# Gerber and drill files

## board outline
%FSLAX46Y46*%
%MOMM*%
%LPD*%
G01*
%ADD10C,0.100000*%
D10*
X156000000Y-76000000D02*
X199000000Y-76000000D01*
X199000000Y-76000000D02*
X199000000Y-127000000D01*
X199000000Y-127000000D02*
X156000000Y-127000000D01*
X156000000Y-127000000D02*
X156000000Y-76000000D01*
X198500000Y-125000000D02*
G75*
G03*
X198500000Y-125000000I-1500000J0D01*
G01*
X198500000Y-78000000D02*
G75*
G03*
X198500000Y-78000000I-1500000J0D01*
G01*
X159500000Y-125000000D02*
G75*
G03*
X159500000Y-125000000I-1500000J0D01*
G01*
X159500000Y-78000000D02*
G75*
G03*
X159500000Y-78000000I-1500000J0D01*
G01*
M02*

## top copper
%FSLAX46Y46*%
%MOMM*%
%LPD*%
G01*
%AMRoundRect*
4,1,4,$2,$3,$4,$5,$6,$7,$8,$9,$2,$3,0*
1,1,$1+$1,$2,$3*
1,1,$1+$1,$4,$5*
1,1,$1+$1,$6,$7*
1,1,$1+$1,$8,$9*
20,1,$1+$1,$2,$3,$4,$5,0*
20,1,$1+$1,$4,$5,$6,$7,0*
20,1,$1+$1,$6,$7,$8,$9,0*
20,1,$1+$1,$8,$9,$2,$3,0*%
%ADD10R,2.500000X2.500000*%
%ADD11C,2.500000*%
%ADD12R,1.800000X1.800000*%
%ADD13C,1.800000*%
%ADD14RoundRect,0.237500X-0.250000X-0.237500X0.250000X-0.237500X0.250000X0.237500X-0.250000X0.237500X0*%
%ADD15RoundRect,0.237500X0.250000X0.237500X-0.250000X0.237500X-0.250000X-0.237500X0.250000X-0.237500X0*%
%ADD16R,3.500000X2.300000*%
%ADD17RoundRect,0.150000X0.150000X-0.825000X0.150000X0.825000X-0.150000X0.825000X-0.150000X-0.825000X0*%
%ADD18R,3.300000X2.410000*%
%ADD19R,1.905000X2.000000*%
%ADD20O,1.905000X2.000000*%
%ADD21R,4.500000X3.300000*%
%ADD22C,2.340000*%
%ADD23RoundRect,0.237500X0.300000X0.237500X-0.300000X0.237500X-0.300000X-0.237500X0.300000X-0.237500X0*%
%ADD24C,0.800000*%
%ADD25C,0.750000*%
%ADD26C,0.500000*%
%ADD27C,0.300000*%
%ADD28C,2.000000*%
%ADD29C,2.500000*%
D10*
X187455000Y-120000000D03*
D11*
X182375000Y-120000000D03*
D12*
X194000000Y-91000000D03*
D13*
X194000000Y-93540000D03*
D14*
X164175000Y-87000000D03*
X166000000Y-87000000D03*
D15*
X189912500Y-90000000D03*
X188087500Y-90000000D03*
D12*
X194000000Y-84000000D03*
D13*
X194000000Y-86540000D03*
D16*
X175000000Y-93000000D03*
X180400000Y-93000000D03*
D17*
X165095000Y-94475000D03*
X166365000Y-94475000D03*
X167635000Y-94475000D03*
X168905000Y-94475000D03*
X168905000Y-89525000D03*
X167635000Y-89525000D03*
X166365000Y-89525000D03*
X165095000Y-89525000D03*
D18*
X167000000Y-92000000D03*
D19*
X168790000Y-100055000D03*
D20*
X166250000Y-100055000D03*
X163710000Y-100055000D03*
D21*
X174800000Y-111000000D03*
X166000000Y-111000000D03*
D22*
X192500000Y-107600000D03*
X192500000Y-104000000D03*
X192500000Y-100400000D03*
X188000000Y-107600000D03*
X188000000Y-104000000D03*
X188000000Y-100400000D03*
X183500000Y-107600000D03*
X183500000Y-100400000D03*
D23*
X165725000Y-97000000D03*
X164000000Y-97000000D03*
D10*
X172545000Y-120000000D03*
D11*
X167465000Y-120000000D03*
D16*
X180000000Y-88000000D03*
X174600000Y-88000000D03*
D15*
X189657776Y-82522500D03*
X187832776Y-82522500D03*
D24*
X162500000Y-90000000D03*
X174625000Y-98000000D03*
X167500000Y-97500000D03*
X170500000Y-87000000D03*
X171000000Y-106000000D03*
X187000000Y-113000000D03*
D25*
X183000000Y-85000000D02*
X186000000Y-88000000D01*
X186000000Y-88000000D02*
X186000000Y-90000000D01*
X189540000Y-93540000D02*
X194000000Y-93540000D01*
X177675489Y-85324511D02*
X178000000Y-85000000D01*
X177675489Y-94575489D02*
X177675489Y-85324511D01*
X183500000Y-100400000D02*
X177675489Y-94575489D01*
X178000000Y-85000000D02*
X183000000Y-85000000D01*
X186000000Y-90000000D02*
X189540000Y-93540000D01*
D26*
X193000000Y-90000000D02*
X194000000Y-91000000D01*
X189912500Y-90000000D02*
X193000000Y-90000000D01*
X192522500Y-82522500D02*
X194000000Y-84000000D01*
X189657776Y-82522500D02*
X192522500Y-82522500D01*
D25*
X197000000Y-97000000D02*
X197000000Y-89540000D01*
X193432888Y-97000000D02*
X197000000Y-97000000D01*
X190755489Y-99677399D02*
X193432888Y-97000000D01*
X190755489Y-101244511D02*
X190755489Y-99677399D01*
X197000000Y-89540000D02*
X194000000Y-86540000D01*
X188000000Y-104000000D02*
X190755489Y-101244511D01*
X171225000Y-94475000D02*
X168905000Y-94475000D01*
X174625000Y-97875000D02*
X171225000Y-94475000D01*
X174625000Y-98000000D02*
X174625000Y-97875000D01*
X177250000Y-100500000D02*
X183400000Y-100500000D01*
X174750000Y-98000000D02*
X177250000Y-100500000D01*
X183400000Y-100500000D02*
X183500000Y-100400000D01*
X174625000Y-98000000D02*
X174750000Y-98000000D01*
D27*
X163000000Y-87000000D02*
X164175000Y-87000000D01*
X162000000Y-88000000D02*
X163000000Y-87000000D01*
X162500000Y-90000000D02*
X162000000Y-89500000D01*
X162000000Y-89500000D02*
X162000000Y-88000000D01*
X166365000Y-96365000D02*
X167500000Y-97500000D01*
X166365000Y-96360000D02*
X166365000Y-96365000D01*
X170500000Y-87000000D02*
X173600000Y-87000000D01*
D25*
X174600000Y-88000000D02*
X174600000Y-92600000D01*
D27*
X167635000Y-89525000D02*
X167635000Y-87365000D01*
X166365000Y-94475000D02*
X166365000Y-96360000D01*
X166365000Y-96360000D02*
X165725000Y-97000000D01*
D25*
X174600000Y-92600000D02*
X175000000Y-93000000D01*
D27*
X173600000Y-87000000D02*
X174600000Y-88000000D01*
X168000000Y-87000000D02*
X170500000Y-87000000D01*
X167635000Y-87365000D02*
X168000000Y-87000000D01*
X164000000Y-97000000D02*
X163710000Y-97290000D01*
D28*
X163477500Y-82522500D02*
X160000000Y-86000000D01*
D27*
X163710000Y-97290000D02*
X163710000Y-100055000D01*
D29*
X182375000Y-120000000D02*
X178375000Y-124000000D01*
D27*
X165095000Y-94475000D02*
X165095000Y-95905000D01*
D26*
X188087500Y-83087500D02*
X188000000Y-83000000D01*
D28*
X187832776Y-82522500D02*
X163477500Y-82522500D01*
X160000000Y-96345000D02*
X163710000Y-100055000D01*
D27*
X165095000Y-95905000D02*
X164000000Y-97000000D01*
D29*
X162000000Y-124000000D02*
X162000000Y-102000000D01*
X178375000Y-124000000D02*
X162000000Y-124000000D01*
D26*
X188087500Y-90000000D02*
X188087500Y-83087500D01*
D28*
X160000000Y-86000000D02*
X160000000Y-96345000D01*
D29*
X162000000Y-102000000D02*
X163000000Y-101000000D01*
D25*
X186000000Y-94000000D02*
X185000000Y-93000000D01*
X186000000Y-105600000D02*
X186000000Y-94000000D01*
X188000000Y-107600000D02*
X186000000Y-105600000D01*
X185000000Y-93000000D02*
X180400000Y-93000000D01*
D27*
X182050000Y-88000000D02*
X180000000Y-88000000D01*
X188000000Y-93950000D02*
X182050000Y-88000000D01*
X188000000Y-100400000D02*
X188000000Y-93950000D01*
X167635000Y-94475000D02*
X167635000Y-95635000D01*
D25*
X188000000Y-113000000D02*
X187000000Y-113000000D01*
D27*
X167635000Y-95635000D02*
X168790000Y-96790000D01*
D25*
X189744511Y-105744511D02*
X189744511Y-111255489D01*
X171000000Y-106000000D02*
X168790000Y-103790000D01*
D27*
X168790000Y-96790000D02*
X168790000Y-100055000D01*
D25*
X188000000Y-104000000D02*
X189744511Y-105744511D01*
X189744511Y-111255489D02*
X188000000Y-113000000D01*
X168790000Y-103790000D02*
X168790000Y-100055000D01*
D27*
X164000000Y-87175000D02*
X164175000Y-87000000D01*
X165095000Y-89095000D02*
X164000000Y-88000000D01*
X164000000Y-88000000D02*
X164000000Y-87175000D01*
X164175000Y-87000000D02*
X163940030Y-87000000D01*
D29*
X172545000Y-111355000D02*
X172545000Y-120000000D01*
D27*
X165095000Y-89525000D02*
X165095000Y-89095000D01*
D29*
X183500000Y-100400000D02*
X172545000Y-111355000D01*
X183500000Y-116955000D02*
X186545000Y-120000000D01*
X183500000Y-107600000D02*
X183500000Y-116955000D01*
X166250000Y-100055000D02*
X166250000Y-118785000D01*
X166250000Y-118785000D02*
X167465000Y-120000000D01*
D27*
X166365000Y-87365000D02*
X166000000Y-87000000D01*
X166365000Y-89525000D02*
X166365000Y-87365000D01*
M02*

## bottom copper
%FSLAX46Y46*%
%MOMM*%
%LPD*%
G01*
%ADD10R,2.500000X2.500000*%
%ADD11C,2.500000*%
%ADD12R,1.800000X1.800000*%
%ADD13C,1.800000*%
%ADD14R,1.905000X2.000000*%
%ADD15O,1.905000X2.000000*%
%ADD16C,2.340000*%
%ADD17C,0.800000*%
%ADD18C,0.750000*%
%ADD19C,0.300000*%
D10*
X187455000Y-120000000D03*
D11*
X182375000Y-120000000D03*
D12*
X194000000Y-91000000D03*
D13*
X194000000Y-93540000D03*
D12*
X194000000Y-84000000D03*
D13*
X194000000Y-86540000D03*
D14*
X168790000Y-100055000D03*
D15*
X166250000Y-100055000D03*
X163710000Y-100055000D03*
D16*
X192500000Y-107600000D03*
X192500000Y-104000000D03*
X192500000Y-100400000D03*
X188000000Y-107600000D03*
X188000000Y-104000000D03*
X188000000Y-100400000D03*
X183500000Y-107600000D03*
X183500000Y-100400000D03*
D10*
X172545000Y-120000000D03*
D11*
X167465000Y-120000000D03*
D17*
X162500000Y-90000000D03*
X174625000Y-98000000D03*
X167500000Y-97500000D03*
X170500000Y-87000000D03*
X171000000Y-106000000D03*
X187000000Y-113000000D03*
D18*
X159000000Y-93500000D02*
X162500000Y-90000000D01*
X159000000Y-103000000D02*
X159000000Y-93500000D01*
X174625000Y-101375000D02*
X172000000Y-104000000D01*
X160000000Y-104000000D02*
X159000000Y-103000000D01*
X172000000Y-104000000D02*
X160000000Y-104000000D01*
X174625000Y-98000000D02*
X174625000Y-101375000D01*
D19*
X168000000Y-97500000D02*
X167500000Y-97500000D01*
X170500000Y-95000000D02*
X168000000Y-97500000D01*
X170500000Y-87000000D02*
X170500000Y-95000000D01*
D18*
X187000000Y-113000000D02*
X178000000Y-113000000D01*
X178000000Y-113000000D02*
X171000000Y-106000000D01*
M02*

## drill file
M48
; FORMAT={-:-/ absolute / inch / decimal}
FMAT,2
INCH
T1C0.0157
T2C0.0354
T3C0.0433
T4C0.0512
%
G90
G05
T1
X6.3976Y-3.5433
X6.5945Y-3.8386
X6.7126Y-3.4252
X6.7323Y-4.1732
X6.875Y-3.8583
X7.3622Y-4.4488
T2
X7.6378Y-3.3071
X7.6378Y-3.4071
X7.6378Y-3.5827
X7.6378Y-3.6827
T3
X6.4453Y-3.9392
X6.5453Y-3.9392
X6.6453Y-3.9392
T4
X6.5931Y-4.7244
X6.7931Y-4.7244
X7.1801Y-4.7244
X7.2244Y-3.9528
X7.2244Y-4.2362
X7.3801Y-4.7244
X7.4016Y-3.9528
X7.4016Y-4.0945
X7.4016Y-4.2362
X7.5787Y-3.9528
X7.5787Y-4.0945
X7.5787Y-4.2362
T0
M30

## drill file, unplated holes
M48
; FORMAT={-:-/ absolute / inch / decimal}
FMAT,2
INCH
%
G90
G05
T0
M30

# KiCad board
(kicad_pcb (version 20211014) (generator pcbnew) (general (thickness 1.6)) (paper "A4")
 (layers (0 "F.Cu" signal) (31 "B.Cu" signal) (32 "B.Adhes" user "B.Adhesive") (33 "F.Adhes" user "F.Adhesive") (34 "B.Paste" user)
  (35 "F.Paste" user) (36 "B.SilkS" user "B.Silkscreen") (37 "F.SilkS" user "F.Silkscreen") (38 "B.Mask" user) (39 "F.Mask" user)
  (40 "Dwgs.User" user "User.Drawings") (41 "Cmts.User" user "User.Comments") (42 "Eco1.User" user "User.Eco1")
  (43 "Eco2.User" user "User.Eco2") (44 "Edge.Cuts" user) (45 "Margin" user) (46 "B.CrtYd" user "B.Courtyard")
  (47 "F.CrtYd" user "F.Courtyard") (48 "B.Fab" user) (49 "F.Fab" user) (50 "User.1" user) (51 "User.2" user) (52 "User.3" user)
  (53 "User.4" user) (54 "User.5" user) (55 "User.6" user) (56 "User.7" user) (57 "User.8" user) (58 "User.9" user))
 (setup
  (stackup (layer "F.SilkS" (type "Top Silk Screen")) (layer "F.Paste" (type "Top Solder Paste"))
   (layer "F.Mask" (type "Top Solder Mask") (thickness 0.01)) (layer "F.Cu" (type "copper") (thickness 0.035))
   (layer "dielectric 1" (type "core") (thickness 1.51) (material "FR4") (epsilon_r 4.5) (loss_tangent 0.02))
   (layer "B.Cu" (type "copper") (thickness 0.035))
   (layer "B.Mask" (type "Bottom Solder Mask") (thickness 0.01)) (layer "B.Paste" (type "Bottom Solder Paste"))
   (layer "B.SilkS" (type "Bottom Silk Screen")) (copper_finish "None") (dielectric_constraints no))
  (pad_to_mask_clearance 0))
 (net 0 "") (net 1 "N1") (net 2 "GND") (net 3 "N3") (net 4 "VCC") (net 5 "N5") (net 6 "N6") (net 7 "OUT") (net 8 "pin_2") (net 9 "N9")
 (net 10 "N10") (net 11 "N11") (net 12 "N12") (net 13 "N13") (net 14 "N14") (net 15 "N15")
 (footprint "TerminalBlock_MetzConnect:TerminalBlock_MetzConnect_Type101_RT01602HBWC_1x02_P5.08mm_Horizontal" (layer "F.Cu")
  (at 187.455 120 180)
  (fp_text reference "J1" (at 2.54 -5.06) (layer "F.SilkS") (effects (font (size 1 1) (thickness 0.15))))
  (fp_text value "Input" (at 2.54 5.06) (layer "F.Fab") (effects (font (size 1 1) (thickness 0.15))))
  (pad "1" thru_hole rect (at 0 0 180) (size 2.5 2.5) (drill 1.3) (layers *.Cu *.Mask) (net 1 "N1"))
  (pad "2" thru_hole circle (at 5.08 0 180) (size 2.5 2.5) (drill 1.3) (layers *.Cu *.Mask) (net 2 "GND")))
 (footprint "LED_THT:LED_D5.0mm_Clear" (layer "F.Cu") (at 194 91 -90)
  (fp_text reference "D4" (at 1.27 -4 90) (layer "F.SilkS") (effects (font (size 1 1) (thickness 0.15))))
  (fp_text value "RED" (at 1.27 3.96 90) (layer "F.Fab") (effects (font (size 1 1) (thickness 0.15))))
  (pad "1" thru_hole rect (at 0 0 270) (size 1.8 1.8) (drill 0.9) (layers *.Cu *.Mask) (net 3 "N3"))
  (pad "2" thru_hole circle (at 2.54 0 270) (size 1.8 1.8) (drill 0.9) (layers *.Cu *.Mask) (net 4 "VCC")))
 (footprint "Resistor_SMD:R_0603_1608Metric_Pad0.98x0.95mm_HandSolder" (layer "F.Cu") (at 165.0875 87)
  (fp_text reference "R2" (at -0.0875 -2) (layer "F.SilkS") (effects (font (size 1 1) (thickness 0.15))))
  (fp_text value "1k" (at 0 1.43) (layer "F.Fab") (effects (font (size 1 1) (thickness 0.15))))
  (pad "1" smd roundrect (at -0.9125 0) (size 0.975 0.95) (layers "F.Cu" "F.Paste" "F.Mask") (roundrect_rratio 0.25) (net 4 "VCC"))
  (pad "2" smd roundrect (at 0.9125 0) (size 0.975 0.95) (layers "F.Cu" "F.Paste" "F.Mask") (roundrect_rratio 0.25) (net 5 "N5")))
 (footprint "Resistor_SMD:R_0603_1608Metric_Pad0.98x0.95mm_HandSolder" (layer "F.Cu") (at 189 90 180)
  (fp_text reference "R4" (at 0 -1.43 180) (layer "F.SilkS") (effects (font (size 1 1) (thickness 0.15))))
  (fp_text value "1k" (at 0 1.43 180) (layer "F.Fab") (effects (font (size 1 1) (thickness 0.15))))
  (pad "1" smd roundrect (at -0.9125 0 180) (size 0.975 0.95) (layers "F.Cu" "F.Paste" "F.Mask") (roundrect_rratio 0.25) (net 3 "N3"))
  (pad "2" smd roundrect (at 0.9125 0 180) (size 0.975 0.95) (layers "F.Cu" "F.Paste" "F.Mask") (roundrect_rratio 0.25) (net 2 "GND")))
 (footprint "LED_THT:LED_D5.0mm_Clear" (layer "F.Cu") (at 194 84 -90)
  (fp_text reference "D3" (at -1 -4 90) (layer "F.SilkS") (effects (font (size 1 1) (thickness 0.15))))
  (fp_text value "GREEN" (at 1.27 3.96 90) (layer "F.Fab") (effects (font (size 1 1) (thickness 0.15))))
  (pad "1" thru_hole rect (at 0 0 270) (size 1.8 1.8) (drill 0.9) (layers *.Cu *.Mask) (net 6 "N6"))
  (pad "2" thru_hole circle (at 2.54 0 270) (size 1.8 1.8) (drill 0.9) (layers *.Cu *.Mask) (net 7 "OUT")))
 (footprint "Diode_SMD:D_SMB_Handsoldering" (layer "F.Cu") (at 177.7 93)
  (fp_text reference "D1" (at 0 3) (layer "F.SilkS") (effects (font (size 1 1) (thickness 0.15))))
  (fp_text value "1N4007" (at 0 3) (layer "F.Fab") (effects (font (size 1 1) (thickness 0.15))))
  (pad "1" smd rect (at -2.7 0) (size 3.5 2.3) (layers "F.Cu" "F.Paste" "F.Mask") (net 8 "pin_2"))
  (pad "2" smd rect (at 2.7 0) (size 3.5 2.3) (layers "F.Cu" "F.Paste" "F.Mask") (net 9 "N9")))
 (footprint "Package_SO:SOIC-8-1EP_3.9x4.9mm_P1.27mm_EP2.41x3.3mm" (layer "F.Cu") (at 167 92 90)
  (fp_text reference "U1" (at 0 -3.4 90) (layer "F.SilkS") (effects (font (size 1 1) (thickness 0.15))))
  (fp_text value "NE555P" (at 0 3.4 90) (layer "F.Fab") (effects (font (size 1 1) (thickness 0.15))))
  (pad "" smd roundrect (at -0.6 -0.825 90) (size 0.97 1.33) (layers "F.Paste") (roundrect_rratio 0.25))
  (pad "" smd roundrect (at 0.6 0.825 90) (size 0.97 1.33) (layers "F.Paste") (roundrect_rratio 0.25))
  (pad "" smd roundrect (at -0.6 0.825 90) (size 0.97 1.33) (layers "F.Paste") (roundrect_rratio 0.25))
  (pad "" smd roundrect (at 0.6 -0.825 90) (size 0.97 1.33) (layers "F.Paste") (roundrect_rratio 0.25))
  (pad "1" smd roundrect (at -2.475 -1.905 90) (size 1.95 0.6) (layers "F.Cu" "F.Paste" "F.Mask") (roundrect_rratio 0.25) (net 2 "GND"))
  (pad "2" smd roundrect (at -2.475 -0.635 90) (size 1.95 0.6) (layers "F.Cu" "F.Paste" "F.Mask") (roundrect_rratio 0.25) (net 8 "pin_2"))
  (pad "3" smd roundrect (at -2.475 0.635 90) (size 1.95 0.6) (layers "F.Cu" "F.Paste" "F.Mask") (roundrect_rratio 0.25) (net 7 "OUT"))
  (pad "4" smd roundrect (at -2.475 1.905 90) (size 1.95 0.6) (layers "F.Cu" "F.Paste" "F.Mask") (roundrect_rratio 0.25) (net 4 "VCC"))
  (pad "5" smd roundrect (at 2.475 1.905 90) (size 1.95 0.6) (layers "F.Cu" "F.Paste" "F.Mask") (roundrect_rratio 0.25) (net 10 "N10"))
  (pad "6" smd roundrect (at 2.475 0.635 90) (size 1.95 0.6) (layers "F.Cu" "F.Paste" "F.Mask") (roundrect_rratio 0.25) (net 8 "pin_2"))
  (pad "7" smd roundrect (at 2.475 -0.635 90) (size 1.95 0.6) (layers "F.Cu" "F.Paste" "F.Mask") (roundrect_rratio 0.25) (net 5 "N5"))
  (pad "8" smd roundrect (at 2.475 -1.905 90) (size 1.95 0.6) (layers "F.Cu" "F.Paste" "F.Mask") (roundrect_rratio 0.25) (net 4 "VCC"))
  (pad "9" smd rect (at 0 0 90) (size 2.41 3.3) (layers "F.Cu" "F.Mask")))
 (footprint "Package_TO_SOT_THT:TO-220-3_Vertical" (layer "F.Cu") (at 168.79 100.055 180)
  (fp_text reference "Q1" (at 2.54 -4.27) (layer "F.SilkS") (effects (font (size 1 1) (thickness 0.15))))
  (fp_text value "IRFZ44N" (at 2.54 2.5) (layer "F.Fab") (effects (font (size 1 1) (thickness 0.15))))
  (pad "1" thru_hole rect (at 0 0 180) (size 1.905 2) (drill 1.1) (layers *.Cu *.Mask) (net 7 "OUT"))
  (pad "2" thru_hole oval (at 2.54 0 180) (size 1.905 2) (drill 1.1) (layers *.Cu *.Mask) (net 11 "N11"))
  (pad "3" thru_hole oval (at 5.08 0 180) (size 1.905 2) (drill 1.1) (layers *.Cu *.Mask) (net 2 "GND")))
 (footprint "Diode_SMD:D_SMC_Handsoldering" (layer "F.Cu") (at 170.4 111 180)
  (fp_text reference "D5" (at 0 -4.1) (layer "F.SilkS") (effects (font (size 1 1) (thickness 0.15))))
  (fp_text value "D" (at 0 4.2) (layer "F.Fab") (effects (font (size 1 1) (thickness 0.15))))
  (pad "1" smd rect (at -4.4 0 270) (size 3.3 4.5) (layers "F.Cu" "F.Paste" "F.Mask") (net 4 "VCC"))
  (pad "2" smd rect (at 4.4 0 270) (size 3.3 4.5) (layers "F.Cu" "F.Paste" "F.Mask") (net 11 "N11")))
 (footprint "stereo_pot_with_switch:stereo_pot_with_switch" (layer "F.Cu") (at 186.5 104)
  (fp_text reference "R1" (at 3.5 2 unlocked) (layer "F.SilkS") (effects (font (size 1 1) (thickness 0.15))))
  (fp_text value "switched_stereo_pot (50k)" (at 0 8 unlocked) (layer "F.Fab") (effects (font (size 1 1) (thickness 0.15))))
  (pad "1" thru_hole circle (at 6 3.6) (size 2.34 2.34) (drill 1.3) (layers *.Cu *.Mask) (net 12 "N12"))
  (pad "2" thru_hole circle (at 6 0) (size 2.34 2.34) (drill 1.3) (layers *.Cu *.Mask) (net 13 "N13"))
  (pad "3" thru_hole circle (at 6 -3.6) (size 2.34 2.34) (drill 1.3) (layers *.Cu *.Mask) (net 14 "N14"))
  (pad "4" thru_hole circle (at 1.5 3.6) (size 2.34 2.34) (drill 1.3) (layers *.Cu *.Mask) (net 9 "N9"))
  (pad "5" thru_hole circle (at 1.5 0) (size 2.34 2.34) (drill 1.3) (layers *.Cu *.Mask) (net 7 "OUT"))
  (pad "6" thru_hole circle (at 1.5 -3.6) (size 2.34 2.34) (drill 1.3) (layers *.Cu *.Mask) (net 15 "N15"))
  (pad "7" thru_hole circle (at -3 3.6) (size 2.34 2.34) (drill 1.3) (layers *.Cu *.Mask) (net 1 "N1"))
  (pad "8" thru_hole circle (at -3 -3.6) (size 2.34 2.34) (drill 1.3) (layers *.Cu *.Mask) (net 4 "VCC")))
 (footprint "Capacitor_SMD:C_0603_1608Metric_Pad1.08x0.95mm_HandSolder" (layer "F.Cu") (at 164.8625 97 180)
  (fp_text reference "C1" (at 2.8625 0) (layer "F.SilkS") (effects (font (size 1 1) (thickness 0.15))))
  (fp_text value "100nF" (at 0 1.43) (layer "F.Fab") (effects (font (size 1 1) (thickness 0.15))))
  (pad "1" smd roundrect (at -0.8625 0 180) (size 1.075 0.95) (layers "F.Cu" "F.Paste" "F.Mask") (roundrect_rratio 0.25) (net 8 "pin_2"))
  (pad "2" smd roundrect (at 0.8625 0 180) (size 1.075 0.95) (layers "F.Cu" "F.Paste" "F.Mask") (roundrect_rratio 0.25) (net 2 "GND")))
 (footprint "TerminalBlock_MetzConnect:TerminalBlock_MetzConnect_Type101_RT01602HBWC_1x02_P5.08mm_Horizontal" (layer "F.Cu")
  (at 172.545 120 180)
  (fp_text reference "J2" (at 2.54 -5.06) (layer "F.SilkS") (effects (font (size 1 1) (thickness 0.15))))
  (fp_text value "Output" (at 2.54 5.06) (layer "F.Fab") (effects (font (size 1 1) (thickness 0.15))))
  (pad "1" thru_hole rect (at 0 0 180) (size 2.5 2.5) (drill 1.3) (layers *.Cu *.Mask) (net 4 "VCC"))
  (pad "2" thru_hole circle (at 5.08 0 180) (size 2.5 2.5) (drill 1.3) (layers *.Cu *.Mask) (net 11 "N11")))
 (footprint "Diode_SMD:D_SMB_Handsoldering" (layer "F.Cu") (at 177.3 88 180)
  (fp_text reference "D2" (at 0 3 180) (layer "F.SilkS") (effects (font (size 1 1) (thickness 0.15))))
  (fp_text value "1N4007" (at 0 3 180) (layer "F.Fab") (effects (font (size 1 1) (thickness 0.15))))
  (pad "1" smd rect (at -2.7 0 180) (size 3.5 2.3) (layers "F.Cu" "F.Paste" "F.Mask") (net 15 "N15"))
  (pad "2" smd rect (at 2.7 0 180) (size 3.5 2.3) (layers "F.Cu" "F.Paste" "F.Mask") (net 8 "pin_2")))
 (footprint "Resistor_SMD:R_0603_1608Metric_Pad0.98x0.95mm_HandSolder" (layer "F.Cu") (at 188.745276 82.5225 180)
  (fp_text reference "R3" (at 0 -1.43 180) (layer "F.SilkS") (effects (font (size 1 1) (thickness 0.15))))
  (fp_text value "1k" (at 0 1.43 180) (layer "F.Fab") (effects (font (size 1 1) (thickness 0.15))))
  (pad "1" smd roundrect (at -0.9125 0 180) (size 0.975 0.95) (layers "F.Cu" "F.Paste" "F.Mask") (roundrect_rratio 0.25) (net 6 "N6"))
  (pad "2" smd roundrect (at 0.9125 0 180) (size 0.975 0.95) (layers "F.Cu" "F.Paste" "F.Mask") (roundrect_rratio 0.25) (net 2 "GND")))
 (gr_rect (start 156 76) (end 199 127) (layer "Edge.Cuts") (width 0.1) (fill none))
 (gr_circle (center 197 125) (end 198.5 125) (layer "Edge.Cuts") (width 0.1) (fill none))
 (gr_circle (center 197 78) (end 198.5 78) (layer "Edge.Cuts") (width 0.1) (fill none))
 (gr_circle (center 158 125) (end 159.5 125) (layer "Edge.Cuts") (width 0.1) (fill none))
 (gr_circle (center 158 78) (end 159.5 78) (layer "Edge.Cuts") (width 0.1) (fill none))
 (segment (start 174.6 88) (end 174.6 92.6) (width 0.75) (layer "F.Cu") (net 8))
 (segment (start 167.635 89.525) (end 167.635 87.365) (width 0.3) (layer "F.Cu") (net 8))
 (segment (start 166.365 94.475) (end 166.365 96.36) (width 0.3) (layer "F.Cu") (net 8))
 (segment (start 166.365 96.36) (end 165.725 97) (width 0.3) (layer "F.Cu") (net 8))
 (segment (start 166.365 96.36) (end 166.365 96.365) (width 0.3) (layer "F.Cu") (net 8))
 (segment (start 174.6 92.6) (end 175 93) (width 0.75) (layer "F.Cu") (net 8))
 (segment (start 173.6 87) (end 174.6 88) (width 0.3) (layer "F.Cu") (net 8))
 (segment (start 168 87) (end 170.5 87) (width 0.3) (layer "F.Cu") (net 8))
 (segment (start 170.5 87) (end 173.6 87) (width 0.3) (layer "F.Cu") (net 8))
 (segment (start 166.365 96.365) (end 167.5 97.5) (width 0.3) (layer "F.Cu") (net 8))
 (segment (start 167.635 87.365) (end 168 87) (width 0.3) (layer "F.Cu") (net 8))
 (via (at 167.5 97.5) (size 0.8) (drill 0.4) (layers "F.Cu" "B.Cu") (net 8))
 (via (at 170.5 87) (size 0.8) (drill 0.4) (layers "F.Cu" "B.Cu") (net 8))
 (segment (start 168 97.5) (end 167.5 97.5) (width 0.3) (layer "B.Cu") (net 8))
 (segment (start 170.5 95) (end 168 97.5) (width 0.3) (layer "B.Cu") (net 8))
 (segment (start 170.5 87) (end 170.5 95) (width 0.3) (layer "B.Cu") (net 8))
 (segment (start 164 97) (end 163.71 97.29) (width 0.3) (layer "F.Cu") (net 2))
 (segment (start 163.4775 82.5225) (end 160 86) (width 2) (layer "F.Cu") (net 2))
 (segment (start 163.71 97.29) (end 163.71 100.055) (width 0.3) (layer "F.Cu") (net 2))
 (segment (start 182.375 120) (end 178.375 124) (width 2.5) (layer "F.Cu") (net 2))
 (segment (start 165.095 94.475) (end 165.095 95.905) (width 0.3) (layer "F.Cu") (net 2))
 (segment (start 188.0875 83.0875) (end 188 83) (width 0.5) (layer "F.Cu") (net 2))
 (segment (start 187.832776 82.5225) (end 163.4775 82.5225) (width 2) (layer "F.Cu") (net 2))
 (segment (start 160 96.345) (end 163.71 100.055) (width 2) (layer "F.Cu") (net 2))
 (segment (start 165.095 95.905) (end 164 97) (width 0.3) (layer "F.Cu") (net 2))
 (segment (start 162 124) (end 162 102) (width 2.5) (layer "F.Cu") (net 2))
 (segment (start 178.375 124) (end 162 124) (width 2.5) (layer "F.Cu") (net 2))
 (segment (start 188.0875 90) (end 188.0875 83.0875) (width 0.5) (layer "F.Cu") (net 2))
 (segment (start 160 86) (end 160 96.345) (width 2) (layer "F.Cu") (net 2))
 (segment (start 162 102) (end 163 101) (width 2.5) (layer "F.Cu") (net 2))
 (segment (start 186 94) (end 185 93) (width 0.75) (layer "F.Cu") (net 9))
 (segment (start 186 105.6) (end 186 94) (width 0.75) (layer "F.Cu") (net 9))
 (segment (start 188 107.6) (end 186 105.6) (width 0.75) (layer "F.Cu") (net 9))
 (segment (start 185 93) (end 180.4 93) (width 0.75) (layer "F.Cu") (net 9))
 (segment (start 182.05 88) (end 180 88) (width 0.3) (layer "F.Cu") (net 15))
 (segment (start 188 93.95) (end 182.05 88) (width 0.3) (layer "F.Cu") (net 15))
 (segment (start 188 100.4) (end 188 93.95) (width 0.3) (layer "F.Cu") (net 15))
 (segment (start 189.657776 82.5225) (end 192.5225 82.5225) (width 0.5) (layer "F.Cu") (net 6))
 (segment (start 192.5225 82.5225) (end 194 84) (width 0.5) (layer "F.Cu") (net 6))
 (segment (start 193.432888 97) (end 197 97) (width 0.75) (layer "F.Cu") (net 7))
 (segment (start 167.635 94.475) (end 167.635 95.635) (width 0.3) (layer "F.Cu") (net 7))
 (segment (start 188 113) (end 187 113) (width 0.75) (layer "F.Cu") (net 7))
 (segment (start 188 104) (end 190.755489 101.244511) (width 0.75) (layer "F.Cu") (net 7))
 (segment (start 167.635 95.635) (end 168.79 96.79) (width 0.3) (layer "F.Cu") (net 7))
 (segment (start 197 97) (end 197 89.54) (width 0.75) (layer "F.Cu") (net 7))
 (segment (start 190.755489 101.244511) (end 190.755489 99.677399) (width 0.75) (layer "F.Cu") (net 7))
 (segment (start 189.744511 105.744511) (end 189.744511 111.255489) (width 0.75) (layer "F.Cu") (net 7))
 (segment (start 171 106) (end 168.79 103.79) (width 0.75) (layer "F.Cu") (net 7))
 (segment (start 168.79 96.79) (end 168.79 100.055) (width 0.3) (layer "F.Cu") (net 7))
 (segment (start 197 89.54) (end 194 86.54) (width 0.75) (layer "F.Cu") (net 7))
 (segment (start 188 104) (end 189.744511 105.744511) (width 0.75) (layer "F.Cu") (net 7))
 (segment (start 189.744511 111.255489) (end 188 113) (width 0.75) (layer "F.Cu") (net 7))
 (segment (start 168.79 103.79) (end 168.79 100.055) (width 0.75) (layer "F.Cu") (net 7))
 (segment (start 190.755489 99.677399) (end 193.432888 97) (width 0.75) (layer "F.Cu") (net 7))
 (via (at 171 106) (size 0.8) (drill 0.4) (layers "F.Cu" "B.Cu") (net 7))
 (via (at 187 113) (size 0.8) (drill 0.4) (layers "F.Cu" "B.Cu") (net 7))
 (segment (start 187 113) (end 178 113) (width 0.75) (layer "B.Cu") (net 7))
 (segment (start 178 113) (end 171 106) (width 0.75) (layer "B.Cu") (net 7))
 (segment (start 193 90) (end 194 91) (width 0.5) (layer "F.Cu") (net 3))
 (segment (start 189.9125 90) (end 193 90) (width 0.5) (layer "F.Cu") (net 3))
 (segment (start 178 85) (end 183 85) (width 0.75) (layer "F.Cu") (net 4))
 (segment (start 174.75 98) (end 177.25 100.5) (width 0.75) (layer "F.Cu") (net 4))
 (segment (start 189.54 93.54) (end 194 93.54) (width 0.75) (layer "F.Cu") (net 4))
 (segment (start 164 87.175) (end 164.175 87) (width 0.3) (layer "F.Cu") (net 4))
 (segment (start 177.675489 85.324511) (end 178 85) (width 0.75) (layer "F.Cu") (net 4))
 (segment (start 186 90) (end 189.54 93.54) (width 0.75) (layer "F.Cu") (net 4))
 (segment (start 162.5 90) (end 162 89.5) (width 0.3) (layer "F.Cu") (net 4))
 (segment (start 174.625 98) (end 174.75 98) (width 0.75) (layer "F.Cu") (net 4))
 (segment (start 165.095 89.095) (end 164 88) (width 0.3) (layer "F.Cu") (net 4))
 (segment (start 183.5 100.4) (end 177.675489 94.575489) (width 0.75) (layer "F.Cu") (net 4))
 (segment (start 163 87) (end 164.175 87) (width 0.3) (layer "F.Cu") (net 4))
 (segment (start 183 85) (end 186 88) (width 0.75) (layer "F.Cu") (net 4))
 (segment (start 164 88) (end 164 87.175) (width 0.3) (layer "F.Cu") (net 4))
 (segment (start 186 88) (end 186 90) (width 0.75) (layer "F.Cu") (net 4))
 (segment (start 164.175 87) (end 163.94003 87) (width 0.3) (layer "F.Cu") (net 4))
 (segment (start 162 88) (end 163 87) (width 0.3) (layer "F.Cu") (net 4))
 (segment (start 183.4 100.5) (end 183.5 100.4) (width 0.75) (layer "F.Cu") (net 4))
 (segment (start 177.675489 94.575489) (end 177.675489 85.324511) (width 0.75) (layer "F.Cu") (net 4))
 (segment (start 172.545 111.355) (end 172.545 120) (width 2.5) (layer "F.Cu") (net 4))
 (segment (start 165.095 89.525) (end 165.095 89.095) (width 0.3) (layer "F.Cu") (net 4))
 (segment (start 174.625 97.875) (end 171.225 94.475) (width 0.75) (layer "F.Cu") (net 4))
 (segment (start 174.625 98) (end 174.625 97.875) (width 0.75) (layer "F.Cu") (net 4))
 (segment (start 183.5 100.4) (end 172.545 111.355) (width 2.5) (layer "F.Cu") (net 4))
 (segment (start 171.225 94.475) (end 168.905 94.475) (width 0.75) (layer "F.Cu") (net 4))
 (segment (start 177.25 100.5) (end 183.4 100.5) (width 0.75) (layer "F.Cu") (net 4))
 (segment (start 162 89.5) (end 162 88) (width 0.3) (layer "F.Cu") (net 4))
 (via (at 174.625 98) (size 0.8) (drill 0.4) (layers "F.Cu" "B.Cu") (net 4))
 (via (at 162.5 90) (size 0.8) (drill 0.4) (layers "F.Cu" "B.Cu") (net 4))
 (segment (start 172 104) (end 160 104) (width 0.75) (layer "B.Cu") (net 4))
 (segment (start 160 104) (end 159 103) (width 0.75) (layer "B.Cu") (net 4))
 (segment (start 174.625 101.375) (end 172 104) (width 0.75) (layer "B.Cu") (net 4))
 (segment (start 159 93.5) (end 162.5 90) (width 0.75) (layer "B.Cu") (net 4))
 (segment (start 159 103) (end 159 93.5) (width 0.75) (layer "B.Cu") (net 4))
 (segment (start 174.625 98) (end 174.625 101.375) (width 0.75) (layer "B.Cu") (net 4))
 (segment (start 183.5 116.955) (end 186.545 120) (width 2.5) (layer "F.Cu") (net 1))
 (segment (start 183.5 107.6) (end 183.5 116.955) (width 2.5) (layer "F.Cu") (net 1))
 (segment (start 166.25 100.055) (end 166.25 118.785) (width 2.5) (layer "F.Cu") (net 11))
 (segment (start 166.25 118.785) (end 167.465 120) (width 2.5) (layer "F.Cu") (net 11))
 (segment (start 166.365 87.365) (end 166 87) (width 0.3) (layer "F.Cu") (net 5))
 (segment (start 166.365 89.525) (end 166.365 87.365) (width 0.3) (layer "F.Cu") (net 5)))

